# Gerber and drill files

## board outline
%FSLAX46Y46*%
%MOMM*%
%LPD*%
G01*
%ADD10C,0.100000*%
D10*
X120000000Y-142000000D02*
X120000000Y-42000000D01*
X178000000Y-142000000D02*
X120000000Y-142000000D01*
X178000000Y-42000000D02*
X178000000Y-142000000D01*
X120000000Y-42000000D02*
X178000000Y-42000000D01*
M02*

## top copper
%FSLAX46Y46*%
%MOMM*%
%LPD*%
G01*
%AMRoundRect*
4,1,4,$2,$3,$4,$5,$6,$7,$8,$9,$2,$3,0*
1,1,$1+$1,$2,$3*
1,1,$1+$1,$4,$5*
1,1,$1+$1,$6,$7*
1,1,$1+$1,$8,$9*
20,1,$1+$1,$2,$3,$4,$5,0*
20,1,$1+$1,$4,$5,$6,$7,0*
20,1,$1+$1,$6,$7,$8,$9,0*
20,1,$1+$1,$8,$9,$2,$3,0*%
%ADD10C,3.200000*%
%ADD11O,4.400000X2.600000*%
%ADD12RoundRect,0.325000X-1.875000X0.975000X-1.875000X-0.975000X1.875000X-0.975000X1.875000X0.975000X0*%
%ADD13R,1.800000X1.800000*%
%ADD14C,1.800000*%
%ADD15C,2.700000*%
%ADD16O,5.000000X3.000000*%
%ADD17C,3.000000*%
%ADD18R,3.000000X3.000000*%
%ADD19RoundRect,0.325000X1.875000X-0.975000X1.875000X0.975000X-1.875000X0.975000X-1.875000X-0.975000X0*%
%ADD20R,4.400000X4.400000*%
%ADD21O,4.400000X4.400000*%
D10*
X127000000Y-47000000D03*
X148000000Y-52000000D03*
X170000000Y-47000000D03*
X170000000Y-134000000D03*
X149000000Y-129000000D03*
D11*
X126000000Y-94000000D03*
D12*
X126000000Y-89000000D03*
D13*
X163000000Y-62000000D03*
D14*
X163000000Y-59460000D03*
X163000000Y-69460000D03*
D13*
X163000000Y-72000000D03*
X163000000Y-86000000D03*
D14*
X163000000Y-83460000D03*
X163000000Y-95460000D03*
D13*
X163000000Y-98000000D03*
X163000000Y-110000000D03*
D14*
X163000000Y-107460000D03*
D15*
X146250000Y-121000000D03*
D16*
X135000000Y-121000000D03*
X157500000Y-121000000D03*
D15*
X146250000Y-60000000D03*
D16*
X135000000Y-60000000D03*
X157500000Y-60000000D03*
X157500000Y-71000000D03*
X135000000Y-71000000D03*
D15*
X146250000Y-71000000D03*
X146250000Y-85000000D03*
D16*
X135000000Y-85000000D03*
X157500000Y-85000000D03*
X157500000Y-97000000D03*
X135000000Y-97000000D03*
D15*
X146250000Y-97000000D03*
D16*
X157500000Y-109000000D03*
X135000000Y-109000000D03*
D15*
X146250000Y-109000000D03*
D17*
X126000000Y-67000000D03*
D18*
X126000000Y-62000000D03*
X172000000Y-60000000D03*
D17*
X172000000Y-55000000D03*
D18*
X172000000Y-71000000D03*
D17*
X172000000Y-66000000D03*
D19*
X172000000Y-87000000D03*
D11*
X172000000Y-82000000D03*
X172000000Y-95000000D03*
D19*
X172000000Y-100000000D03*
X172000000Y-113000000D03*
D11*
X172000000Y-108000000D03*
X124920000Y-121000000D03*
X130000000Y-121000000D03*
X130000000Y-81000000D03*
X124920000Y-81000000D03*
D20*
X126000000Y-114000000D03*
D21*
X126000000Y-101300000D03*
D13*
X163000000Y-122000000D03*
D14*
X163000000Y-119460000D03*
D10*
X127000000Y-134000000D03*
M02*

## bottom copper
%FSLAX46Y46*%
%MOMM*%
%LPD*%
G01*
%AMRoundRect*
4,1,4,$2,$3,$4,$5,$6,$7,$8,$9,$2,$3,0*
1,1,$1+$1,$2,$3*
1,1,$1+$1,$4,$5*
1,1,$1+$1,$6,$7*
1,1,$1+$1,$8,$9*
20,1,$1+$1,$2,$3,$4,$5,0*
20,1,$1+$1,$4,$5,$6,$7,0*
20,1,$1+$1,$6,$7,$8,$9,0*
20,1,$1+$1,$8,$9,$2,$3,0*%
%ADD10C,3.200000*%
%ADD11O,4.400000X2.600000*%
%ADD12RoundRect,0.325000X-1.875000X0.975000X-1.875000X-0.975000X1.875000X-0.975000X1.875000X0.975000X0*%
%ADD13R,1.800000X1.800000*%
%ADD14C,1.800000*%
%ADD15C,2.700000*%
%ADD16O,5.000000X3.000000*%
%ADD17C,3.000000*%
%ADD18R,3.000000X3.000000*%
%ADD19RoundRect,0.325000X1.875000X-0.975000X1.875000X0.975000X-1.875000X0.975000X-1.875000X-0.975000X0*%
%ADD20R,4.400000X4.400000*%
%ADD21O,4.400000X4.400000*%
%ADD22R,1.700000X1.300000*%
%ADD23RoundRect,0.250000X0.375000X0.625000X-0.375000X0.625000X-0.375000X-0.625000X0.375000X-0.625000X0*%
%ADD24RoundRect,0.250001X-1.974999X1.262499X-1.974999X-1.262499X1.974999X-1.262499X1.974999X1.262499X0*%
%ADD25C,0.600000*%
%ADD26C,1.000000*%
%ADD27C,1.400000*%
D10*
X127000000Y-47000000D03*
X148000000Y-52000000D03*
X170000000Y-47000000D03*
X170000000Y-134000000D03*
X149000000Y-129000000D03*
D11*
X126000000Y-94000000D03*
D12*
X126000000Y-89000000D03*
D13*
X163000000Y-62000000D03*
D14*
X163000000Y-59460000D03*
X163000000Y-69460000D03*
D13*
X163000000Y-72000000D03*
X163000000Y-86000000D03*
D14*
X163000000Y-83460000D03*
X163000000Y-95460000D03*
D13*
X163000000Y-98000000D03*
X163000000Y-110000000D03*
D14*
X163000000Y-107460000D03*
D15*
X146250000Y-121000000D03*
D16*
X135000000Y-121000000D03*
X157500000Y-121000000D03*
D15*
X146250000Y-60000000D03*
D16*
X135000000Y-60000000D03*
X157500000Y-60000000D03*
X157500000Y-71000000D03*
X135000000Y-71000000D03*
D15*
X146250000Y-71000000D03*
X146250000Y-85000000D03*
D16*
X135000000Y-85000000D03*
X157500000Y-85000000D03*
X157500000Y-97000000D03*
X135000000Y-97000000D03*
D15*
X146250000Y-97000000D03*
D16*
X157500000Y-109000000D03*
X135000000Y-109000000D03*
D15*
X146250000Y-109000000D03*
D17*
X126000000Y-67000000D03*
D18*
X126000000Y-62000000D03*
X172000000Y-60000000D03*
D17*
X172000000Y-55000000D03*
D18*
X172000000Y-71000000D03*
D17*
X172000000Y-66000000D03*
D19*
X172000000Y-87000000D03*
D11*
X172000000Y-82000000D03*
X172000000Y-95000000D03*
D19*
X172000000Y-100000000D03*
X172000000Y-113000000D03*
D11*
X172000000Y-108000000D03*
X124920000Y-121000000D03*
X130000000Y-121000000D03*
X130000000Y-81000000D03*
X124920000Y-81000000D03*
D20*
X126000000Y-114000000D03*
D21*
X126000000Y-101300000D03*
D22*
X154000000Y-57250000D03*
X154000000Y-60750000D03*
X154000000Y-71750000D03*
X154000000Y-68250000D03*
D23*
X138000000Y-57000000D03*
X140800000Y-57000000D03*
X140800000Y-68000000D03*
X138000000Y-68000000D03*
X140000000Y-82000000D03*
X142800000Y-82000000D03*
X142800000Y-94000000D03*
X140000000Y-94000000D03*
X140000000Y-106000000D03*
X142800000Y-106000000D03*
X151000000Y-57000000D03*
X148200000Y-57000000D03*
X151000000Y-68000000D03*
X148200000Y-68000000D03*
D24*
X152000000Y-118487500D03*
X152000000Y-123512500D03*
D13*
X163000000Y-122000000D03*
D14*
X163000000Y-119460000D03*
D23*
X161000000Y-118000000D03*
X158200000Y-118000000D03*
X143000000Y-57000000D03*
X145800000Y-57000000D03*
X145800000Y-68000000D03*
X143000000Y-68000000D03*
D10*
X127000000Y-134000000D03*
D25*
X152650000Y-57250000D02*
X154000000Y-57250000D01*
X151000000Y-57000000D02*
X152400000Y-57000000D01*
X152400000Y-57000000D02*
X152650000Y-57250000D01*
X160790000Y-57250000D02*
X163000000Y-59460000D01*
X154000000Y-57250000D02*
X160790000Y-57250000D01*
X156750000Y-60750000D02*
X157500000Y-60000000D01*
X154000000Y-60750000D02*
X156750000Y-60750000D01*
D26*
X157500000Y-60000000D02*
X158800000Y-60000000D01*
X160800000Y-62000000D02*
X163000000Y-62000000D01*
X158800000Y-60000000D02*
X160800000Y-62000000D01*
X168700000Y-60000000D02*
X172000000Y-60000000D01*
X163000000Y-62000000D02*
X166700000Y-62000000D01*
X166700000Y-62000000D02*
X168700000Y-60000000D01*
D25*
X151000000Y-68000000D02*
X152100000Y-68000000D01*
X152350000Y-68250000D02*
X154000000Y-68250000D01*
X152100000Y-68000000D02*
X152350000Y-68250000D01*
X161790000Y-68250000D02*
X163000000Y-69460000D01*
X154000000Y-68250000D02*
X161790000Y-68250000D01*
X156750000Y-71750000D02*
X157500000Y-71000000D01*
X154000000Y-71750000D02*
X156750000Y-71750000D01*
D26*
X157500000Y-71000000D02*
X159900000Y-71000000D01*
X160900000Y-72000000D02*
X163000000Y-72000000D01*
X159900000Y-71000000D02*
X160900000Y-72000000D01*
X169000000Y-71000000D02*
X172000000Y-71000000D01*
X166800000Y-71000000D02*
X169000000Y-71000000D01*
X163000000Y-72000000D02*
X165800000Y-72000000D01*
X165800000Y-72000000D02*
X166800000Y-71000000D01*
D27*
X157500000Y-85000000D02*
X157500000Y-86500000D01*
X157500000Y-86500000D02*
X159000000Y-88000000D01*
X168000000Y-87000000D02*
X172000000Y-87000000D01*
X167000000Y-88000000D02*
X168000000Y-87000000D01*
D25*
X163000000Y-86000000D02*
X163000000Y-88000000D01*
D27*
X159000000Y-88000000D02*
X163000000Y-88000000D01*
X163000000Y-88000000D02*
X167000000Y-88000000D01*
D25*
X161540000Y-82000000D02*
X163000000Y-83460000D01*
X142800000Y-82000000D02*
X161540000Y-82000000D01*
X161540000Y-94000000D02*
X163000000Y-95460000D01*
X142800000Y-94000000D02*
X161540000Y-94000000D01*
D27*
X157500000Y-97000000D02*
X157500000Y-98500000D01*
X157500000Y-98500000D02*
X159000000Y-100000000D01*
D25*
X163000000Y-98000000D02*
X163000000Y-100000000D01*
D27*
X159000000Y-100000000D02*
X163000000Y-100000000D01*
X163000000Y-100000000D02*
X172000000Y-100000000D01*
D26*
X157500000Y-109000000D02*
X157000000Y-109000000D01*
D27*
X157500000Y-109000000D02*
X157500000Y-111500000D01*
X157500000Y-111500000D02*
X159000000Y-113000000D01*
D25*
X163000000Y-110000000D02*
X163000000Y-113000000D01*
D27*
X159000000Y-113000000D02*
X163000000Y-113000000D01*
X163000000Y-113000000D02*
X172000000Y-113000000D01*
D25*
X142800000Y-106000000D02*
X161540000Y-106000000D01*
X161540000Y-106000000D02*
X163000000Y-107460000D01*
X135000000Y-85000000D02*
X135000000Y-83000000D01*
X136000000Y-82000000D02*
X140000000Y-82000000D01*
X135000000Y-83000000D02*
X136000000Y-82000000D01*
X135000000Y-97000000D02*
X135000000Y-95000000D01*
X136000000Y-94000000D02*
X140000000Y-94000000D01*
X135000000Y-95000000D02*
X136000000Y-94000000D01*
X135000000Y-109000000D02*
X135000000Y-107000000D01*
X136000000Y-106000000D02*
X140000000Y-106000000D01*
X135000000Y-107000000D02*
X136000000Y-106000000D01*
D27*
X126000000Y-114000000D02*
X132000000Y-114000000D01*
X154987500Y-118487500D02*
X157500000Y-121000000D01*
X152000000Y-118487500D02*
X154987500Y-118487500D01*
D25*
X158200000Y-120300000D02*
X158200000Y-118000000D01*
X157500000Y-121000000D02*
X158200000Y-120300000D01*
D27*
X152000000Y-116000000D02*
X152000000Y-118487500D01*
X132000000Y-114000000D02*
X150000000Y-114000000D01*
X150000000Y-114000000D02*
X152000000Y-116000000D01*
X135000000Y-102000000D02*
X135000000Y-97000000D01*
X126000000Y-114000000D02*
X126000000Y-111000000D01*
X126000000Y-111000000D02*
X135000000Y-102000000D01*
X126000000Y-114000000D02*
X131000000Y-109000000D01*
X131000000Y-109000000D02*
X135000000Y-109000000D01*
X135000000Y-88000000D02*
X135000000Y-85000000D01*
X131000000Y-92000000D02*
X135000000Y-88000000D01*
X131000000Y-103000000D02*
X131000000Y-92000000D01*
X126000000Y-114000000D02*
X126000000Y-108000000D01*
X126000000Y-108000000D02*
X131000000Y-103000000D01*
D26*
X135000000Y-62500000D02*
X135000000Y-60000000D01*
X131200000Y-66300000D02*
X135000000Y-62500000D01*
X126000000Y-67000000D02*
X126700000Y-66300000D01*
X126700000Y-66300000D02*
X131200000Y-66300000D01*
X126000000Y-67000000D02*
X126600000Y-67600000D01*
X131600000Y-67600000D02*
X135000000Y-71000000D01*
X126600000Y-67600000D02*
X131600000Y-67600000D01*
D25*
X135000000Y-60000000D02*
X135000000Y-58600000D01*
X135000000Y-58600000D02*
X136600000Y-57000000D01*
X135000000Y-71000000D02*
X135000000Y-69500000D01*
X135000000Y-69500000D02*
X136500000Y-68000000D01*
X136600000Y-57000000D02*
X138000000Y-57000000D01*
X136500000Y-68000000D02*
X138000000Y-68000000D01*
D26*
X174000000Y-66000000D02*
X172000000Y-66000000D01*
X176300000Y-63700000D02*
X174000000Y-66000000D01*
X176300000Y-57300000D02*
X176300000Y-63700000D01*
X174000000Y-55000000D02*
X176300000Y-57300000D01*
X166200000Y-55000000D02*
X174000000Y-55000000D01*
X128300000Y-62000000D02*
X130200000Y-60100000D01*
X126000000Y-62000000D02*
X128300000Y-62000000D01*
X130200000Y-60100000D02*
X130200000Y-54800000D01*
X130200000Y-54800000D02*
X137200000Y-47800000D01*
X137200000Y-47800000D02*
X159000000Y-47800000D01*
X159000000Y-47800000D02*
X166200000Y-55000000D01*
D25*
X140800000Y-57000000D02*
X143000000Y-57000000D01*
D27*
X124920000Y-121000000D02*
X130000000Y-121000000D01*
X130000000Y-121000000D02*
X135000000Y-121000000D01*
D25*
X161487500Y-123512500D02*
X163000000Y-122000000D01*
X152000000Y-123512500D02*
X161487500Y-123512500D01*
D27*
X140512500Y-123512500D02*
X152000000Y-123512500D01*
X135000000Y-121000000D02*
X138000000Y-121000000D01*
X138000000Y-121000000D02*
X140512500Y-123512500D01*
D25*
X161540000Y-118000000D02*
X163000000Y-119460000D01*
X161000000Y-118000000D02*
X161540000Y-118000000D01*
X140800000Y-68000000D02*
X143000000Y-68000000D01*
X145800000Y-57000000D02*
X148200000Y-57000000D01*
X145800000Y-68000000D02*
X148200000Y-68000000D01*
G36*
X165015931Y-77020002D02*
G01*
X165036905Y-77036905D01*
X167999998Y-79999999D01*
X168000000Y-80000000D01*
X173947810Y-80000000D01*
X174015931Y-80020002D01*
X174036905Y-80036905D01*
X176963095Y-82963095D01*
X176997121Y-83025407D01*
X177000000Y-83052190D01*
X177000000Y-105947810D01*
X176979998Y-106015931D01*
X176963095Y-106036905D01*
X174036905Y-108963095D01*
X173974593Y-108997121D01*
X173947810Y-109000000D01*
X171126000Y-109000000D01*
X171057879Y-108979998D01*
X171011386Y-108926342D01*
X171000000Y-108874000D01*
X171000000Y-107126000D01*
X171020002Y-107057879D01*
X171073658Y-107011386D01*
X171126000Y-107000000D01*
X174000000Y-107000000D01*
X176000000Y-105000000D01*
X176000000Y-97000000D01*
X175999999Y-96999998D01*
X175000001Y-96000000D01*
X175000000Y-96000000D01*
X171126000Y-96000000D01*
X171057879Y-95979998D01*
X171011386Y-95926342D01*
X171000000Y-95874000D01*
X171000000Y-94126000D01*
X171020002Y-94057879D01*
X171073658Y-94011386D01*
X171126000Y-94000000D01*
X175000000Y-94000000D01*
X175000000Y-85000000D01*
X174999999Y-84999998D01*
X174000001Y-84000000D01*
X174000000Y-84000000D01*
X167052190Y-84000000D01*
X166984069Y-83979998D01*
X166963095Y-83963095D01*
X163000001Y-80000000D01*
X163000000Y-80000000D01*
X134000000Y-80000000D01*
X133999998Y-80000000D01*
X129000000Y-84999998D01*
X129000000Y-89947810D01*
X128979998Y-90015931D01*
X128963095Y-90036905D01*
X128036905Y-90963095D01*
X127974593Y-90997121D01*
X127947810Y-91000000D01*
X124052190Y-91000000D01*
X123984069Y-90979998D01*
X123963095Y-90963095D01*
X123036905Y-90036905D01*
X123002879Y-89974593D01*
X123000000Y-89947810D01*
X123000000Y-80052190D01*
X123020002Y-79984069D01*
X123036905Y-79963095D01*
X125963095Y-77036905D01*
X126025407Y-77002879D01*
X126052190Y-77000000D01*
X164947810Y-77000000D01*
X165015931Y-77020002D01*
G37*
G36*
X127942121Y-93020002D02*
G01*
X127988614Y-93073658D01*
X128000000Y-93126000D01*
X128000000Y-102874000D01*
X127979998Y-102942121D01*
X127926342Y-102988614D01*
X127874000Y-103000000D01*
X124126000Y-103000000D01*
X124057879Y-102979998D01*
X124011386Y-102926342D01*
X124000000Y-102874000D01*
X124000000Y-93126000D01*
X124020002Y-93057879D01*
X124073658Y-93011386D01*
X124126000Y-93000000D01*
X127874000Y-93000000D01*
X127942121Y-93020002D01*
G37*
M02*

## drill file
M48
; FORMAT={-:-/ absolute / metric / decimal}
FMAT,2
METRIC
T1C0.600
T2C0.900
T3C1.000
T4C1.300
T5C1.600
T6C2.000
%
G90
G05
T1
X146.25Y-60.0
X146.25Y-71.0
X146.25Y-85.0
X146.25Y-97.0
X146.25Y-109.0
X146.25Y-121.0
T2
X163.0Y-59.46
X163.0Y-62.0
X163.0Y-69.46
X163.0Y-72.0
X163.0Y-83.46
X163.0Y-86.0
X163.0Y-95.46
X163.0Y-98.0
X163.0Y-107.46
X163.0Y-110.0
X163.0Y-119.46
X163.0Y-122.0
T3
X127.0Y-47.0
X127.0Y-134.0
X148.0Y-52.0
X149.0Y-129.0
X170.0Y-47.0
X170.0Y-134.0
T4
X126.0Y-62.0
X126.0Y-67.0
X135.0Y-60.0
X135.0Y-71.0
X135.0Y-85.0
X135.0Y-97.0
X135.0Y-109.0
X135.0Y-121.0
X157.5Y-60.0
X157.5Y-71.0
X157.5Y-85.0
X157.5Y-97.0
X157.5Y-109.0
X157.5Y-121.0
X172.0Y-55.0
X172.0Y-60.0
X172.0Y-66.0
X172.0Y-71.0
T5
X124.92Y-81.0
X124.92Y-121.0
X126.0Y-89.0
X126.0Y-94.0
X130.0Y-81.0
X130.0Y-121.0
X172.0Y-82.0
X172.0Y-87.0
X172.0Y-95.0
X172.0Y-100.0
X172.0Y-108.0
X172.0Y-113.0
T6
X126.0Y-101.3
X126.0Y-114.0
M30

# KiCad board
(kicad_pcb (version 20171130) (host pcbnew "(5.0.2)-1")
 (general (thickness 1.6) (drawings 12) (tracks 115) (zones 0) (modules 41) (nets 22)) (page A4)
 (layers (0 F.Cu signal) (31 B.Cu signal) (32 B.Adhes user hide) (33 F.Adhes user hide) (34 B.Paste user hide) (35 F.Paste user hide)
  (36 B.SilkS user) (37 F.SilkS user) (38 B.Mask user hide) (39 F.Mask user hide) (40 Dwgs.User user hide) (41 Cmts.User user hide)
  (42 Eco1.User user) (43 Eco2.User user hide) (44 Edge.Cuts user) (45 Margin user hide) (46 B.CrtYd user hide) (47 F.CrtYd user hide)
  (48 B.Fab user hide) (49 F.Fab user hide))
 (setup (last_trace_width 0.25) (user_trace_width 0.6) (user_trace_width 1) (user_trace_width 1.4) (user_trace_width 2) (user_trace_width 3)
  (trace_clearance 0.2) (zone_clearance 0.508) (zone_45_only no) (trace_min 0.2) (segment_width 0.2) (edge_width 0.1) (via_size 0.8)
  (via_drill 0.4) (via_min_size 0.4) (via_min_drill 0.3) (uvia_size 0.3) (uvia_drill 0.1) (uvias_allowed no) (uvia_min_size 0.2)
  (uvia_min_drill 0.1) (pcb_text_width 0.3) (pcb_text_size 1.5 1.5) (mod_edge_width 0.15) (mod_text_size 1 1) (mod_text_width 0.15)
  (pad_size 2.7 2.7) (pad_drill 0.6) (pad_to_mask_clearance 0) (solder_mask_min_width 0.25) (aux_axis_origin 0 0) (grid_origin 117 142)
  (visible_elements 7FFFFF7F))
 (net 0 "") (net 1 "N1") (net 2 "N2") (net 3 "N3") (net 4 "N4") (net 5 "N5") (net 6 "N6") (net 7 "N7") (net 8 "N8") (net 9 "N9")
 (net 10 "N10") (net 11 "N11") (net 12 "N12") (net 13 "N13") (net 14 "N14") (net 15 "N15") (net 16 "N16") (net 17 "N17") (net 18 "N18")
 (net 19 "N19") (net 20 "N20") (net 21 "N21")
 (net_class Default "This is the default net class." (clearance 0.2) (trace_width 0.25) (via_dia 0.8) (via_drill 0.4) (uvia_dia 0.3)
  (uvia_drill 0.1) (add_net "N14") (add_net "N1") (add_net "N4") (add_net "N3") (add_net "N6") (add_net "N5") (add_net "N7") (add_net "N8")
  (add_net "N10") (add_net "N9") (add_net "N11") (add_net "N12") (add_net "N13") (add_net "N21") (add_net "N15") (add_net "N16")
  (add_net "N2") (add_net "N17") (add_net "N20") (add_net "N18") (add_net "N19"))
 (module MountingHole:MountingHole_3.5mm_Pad (layer F.Cu) (at 127 47)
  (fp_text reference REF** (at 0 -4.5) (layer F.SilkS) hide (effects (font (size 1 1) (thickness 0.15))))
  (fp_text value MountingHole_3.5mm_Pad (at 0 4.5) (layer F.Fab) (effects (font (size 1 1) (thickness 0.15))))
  (pad 1 thru_hole circle (at 0 0) (size 3.2 3.2) (drill 1) (layers *.Cu *.Mask)))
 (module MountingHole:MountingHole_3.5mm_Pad (layer F.Cu) (at 148 52)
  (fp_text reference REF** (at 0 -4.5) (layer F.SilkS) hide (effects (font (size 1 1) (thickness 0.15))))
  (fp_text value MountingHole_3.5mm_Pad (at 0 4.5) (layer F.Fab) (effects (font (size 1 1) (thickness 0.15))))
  (pad 1 thru_hole circle (at 0 0) (size 3.2 3.2) (drill 1) (layers *.Cu *.Mask)))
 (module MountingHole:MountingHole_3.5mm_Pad (layer F.Cu) (at 170 47)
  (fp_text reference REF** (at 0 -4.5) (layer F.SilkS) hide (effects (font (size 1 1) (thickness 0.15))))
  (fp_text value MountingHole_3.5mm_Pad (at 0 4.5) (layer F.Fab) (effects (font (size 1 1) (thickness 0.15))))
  (pad 1 thru_hole circle (at 0 0) (size 3.2 3.2) (drill 1) (layers *.Cu *.Mask)))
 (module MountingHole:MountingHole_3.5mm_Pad (layer F.Cu) (at 170 134)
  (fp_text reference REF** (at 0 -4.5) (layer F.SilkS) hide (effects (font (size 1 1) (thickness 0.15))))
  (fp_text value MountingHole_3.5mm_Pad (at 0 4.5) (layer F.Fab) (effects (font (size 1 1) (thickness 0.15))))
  (pad 1 thru_hole circle (at 0 0) (size 3.2 3.2) (drill 1) (layers *.Cu *.Mask)))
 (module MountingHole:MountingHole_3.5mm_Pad (layer F.Cu) (at 149 129)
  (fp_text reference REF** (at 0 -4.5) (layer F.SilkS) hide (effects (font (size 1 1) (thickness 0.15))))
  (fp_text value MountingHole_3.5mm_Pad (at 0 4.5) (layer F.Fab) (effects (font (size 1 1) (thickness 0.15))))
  (pad 1 thru_hole circle (at 0 0) (size 3.2 3.2) (drill 1) (layers *.Cu *.Mask)))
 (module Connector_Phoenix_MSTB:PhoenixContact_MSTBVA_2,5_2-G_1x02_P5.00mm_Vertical (layer F.Cu) (at 126 89 270)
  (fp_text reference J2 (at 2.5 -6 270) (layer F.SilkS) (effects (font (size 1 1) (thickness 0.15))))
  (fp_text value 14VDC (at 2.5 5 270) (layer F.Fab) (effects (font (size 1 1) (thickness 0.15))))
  (pad 2 thru_hole oval (at 5 0 270) (size 2.6 4.4) (drill 1.6) (layers *.Cu *.Mask) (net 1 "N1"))
  (pad 1 thru_hole roundrect (at 0 0 270) (size 2.6 4.4) (drill 1.6) (layers *.Cu *.Mask) (roundrect_rratio 0.125) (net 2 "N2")))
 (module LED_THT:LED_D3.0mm (layer F.Cu) (at 163 62 90)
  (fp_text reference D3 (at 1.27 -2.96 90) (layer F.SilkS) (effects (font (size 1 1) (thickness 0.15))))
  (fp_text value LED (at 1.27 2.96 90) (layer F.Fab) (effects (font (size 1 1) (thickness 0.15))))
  (pad 1 thru_hole rect (at 0 0 90) (size 1.8 1.8) (drill 0.9) (layers *.Cu *.Mask) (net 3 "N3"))
  (pad 2 thru_hole circle (at 2.54 0 90) (size 1.8 1.8) (drill 0.9) (layers *.Cu *.Mask) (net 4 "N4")))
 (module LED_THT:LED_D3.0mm (layer F.Cu) (at 163 72 90)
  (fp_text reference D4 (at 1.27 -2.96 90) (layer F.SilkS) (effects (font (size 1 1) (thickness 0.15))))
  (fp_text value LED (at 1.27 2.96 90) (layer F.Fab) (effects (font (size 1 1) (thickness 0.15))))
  (pad 2 thru_hole circle (at 2.54 0 90) (size 1.8 1.8) (drill 0.9) (layers *.Cu *.Mask) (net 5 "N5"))
  (pad 1 thru_hole rect (at 0 0 90) (size 1.8 1.8) (drill 0.9) (layers *.Cu *.Mask) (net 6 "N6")))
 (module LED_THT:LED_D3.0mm (layer F.Cu) (at 163 86 90)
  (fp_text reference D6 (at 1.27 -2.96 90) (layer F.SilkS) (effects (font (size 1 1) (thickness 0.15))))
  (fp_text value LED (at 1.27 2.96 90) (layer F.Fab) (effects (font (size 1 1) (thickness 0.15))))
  (pad 1 thru_hole rect (at 0 0 90) (size 1.8 1.8) (drill 0.9) (layers *.Cu *.Mask) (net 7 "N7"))
  (pad 2 thru_hole circle (at 2.54 0 90) (size 1.8 1.8) (drill 0.9) (layers *.Cu *.Mask) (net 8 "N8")))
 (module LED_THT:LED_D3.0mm (layer F.Cu) (at 163 98 90)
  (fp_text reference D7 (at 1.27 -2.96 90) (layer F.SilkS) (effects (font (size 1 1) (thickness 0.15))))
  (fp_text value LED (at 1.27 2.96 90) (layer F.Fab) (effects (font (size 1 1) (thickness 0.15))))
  (pad 2 thru_hole circle (at 2.54 0 90) (size 1.8 1.8) (drill 0.9) (layers *.Cu *.Mask) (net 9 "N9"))
  (pad 1 thru_hole rect (at 0 0 90) (size 1.8 1.8) (drill 0.9) (layers *.Cu *.Mask) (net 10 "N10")))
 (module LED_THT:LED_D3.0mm (layer F.Cu) (at 163 110 90)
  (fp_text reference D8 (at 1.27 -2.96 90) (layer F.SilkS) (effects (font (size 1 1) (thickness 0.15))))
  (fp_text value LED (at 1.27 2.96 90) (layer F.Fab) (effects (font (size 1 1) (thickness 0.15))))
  (pad 1 thru_hole rect (at 0 0 90) (size 1.8 1.8) (drill 0.9) (layers *.Cu *.Mask) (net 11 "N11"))
  (pad 2 thru_hole circle (at 2.54 0 90) (size 1.8 1.8) (drill 0.9) (layers *.Cu *.Mask) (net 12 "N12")))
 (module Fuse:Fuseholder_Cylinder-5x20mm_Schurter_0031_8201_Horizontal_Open (layer F.Cu) (at 157.5 121 180)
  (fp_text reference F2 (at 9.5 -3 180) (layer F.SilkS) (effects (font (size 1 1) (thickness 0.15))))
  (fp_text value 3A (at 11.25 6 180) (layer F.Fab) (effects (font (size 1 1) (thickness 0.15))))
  (pad "" thru_hole circle (at 11.25 0 180) (size 2.7 2.7) (drill 0.6) (layers *.Cu *.Mask))
  (pad 2 thru_hole oval (at 22.5 0 180) (size 5 3) (drill 1.3) (layers *.Cu *.Mask) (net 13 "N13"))
  (pad 1 thru_hole oval (at 0 0 180) (size 5 3) (drill 1.3) (layers *.Cu *.Mask) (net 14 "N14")))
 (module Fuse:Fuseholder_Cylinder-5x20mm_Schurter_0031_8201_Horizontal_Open (layer F.Cu) (at 157.5 60 180)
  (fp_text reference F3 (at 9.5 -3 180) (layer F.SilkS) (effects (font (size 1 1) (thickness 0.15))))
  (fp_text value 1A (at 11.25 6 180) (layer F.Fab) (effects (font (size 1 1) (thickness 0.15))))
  (pad "" thru_hole circle (at 11.25 0 180) (size 2.7 2.7) (drill 0.6) (layers *.Cu *.Mask))
  (pad 2 thru_hole oval (at 22.5 0 180) (size 5 3) (drill 1.3) (layers *.Cu *.Mask) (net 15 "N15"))
  (pad 1 thru_hole oval (at 0 0 180) (size 5 3) (drill 1.3) (layers *.Cu *.Mask) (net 3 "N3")))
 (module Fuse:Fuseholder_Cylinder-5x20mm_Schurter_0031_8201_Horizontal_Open (layer F.Cu) (at 157.5 71 180)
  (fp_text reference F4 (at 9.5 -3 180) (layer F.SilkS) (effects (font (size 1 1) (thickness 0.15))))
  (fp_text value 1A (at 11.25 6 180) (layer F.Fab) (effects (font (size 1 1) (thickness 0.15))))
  (pad 1 thru_hole oval (at 0 0 180) (size 5 3) (drill 1.3) (layers *.Cu *.Mask) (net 6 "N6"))
  (pad 2 thru_hole oval (at 22.5 0 180) (size 5 3) (drill 1.3) (layers *.Cu *.Mask) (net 15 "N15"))
  (pad "" thru_hole circle (at 11.25 0 180) (size 2.7 2.7) (drill 0.6) (layers *.Cu *.Mask)))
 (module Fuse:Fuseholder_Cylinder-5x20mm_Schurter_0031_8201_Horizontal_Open (layer F.Cu) (at 157.5 85 180)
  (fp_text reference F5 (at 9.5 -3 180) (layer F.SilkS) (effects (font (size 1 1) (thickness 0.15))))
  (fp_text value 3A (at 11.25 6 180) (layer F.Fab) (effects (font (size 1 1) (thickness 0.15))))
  (pad "" thru_hole circle (at 11.25 0 180) (size 2.7 2.7) (drill 0.6) (layers *.Cu *.Mask))
  (pad 2 thru_hole oval (at 22.5 0 180) (size 5 3) (drill 1.3) (layers *.Cu *.Mask) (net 14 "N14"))
  (pad 1 thru_hole oval (at 0 0 180) (size 5 3) (drill 1.3) (layers *.Cu *.Mask) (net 7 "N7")))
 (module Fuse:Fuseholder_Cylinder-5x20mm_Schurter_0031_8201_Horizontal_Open (layer F.Cu) (at 157.5 97 180)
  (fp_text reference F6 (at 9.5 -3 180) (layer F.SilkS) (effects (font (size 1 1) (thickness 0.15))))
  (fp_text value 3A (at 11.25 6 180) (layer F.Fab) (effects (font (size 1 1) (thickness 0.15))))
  (pad 1 thru_hole oval (at 0 0 180) (size 5 3) (drill 1.3) (layers *.Cu *.Mask) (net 10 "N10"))
  (pad 2 thru_hole oval (at 22.5 0 180) (size 5 3) (drill 1.3) (layers *.Cu *.Mask) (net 14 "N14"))
  (pad "" thru_hole circle (at 11.25 0 180) (size 2.7 2.7) (drill 0.6) (layers *.Cu *.Mask)))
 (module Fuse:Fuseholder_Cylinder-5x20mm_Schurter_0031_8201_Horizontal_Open (layer F.Cu) (at 157.5 109 180)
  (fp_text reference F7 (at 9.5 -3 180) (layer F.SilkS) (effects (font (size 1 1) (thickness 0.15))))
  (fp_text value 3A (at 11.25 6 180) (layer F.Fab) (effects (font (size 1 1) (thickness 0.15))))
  (pad 1 thru_hole oval (at 0 0 180) (size 5 3) (drill 1.3) (layers *.Cu *.Mask) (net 11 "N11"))
  (pad 2 thru_hole oval (at 22.5 0 180) (size 5 3) (drill 1.3) (layers *.Cu *.Mask) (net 14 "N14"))
  (pad "" thru_hole circle (at 11.25 0 180) (size 2.7 2.7) (drill 0.6) (layers *.Cu *.Mask)))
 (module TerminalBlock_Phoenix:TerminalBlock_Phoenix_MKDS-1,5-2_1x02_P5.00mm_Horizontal (layer F.Cu) (at 126 62 270)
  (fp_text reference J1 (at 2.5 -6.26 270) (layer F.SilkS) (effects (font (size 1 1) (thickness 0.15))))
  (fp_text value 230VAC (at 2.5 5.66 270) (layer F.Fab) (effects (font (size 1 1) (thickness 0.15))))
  (pad 2 thru_hole circle (at 5 0 270) (size 3 3) (drill 1.3) (layers *.Cu *.Mask) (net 15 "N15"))
  (pad 1 thru_hole rect (at 0 0 270) (size 3 3) (drill 1.3) (layers *.Cu *.Mask) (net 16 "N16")))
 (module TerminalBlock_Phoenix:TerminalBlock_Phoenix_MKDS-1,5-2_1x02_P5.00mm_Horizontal (layer F.Cu) (at 172 60 90)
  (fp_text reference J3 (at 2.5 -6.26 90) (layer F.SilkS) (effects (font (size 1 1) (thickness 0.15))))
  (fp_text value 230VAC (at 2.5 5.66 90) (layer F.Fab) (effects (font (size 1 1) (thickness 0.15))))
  (pad 1 thru_hole rect (at 0 0 90) (size 3 3) (drill 1.3) (layers *.Cu *.Mask) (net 3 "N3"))
  (pad 2 thru_hole circle (at 5 0 90) (size 3 3) (drill 1.3) (layers *.Cu *.Mask) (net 16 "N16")))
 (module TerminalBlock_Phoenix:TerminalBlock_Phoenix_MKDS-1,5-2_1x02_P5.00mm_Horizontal (layer F.Cu) (at 172 71 90)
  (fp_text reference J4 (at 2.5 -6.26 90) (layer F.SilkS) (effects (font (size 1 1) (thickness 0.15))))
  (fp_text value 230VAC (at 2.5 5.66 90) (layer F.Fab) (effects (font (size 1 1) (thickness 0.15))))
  (pad 1 thru_hole rect (at 0 0 90) (size 3 3) (drill 1.3) (layers *.Cu *.Mask) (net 6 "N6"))
  (pad 2 thru_hole circle (at 5 0 90) (size 3 3) (drill 1.3) (layers *.Cu *.Mask) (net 16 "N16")))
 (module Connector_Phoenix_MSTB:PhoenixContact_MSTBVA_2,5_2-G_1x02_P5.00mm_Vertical (layer F.Cu) (at 172 87 90)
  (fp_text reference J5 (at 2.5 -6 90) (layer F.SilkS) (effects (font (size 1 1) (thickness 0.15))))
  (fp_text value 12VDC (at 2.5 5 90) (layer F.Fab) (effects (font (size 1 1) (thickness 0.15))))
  (pad 1 thru_hole roundrect (at 0 0 90) (size 2.6 4.4) (drill 1.6) (layers *.Cu *.Mask) (roundrect_rratio 0.125) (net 7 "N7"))
  (pad 2 thru_hole oval (at 5 0 90) (size 2.6 4.4) (drill 1.6) (layers *.Cu *.Mask) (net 2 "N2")))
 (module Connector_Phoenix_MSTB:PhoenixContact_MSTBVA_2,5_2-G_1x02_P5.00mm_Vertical (layer F.Cu) (at 172 100 90)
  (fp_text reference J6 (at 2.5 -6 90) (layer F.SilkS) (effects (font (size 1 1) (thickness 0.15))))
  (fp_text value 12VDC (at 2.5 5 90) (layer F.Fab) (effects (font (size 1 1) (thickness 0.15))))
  (pad 2 thru_hole oval (at 5 0 90) (size 2.6 4.4) (drill 1.6) (layers *.Cu *.Mask) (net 2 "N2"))
  (pad 1 thru_hole roundrect (at 0 0 90) (size 2.6 4.4) (drill 1.6) (layers *.Cu *.Mask) (roundrect_rratio 0.125) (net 10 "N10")))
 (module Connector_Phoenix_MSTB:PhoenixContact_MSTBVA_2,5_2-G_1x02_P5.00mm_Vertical (layer F.Cu) (at 172 113 90)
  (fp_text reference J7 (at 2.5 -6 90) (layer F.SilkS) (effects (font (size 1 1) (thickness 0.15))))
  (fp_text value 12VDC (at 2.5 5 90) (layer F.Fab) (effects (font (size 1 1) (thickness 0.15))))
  (pad 1 thru_hole roundrect (at 0 0 90) (size 2.6 4.4) (drill 1.6) (layers *.Cu *.Mask) (roundrect_rratio 0.125) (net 11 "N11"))
  (pad 2 thru_hole oval (at 5 0 90) (size 2.6 4.4) (drill 1.6) (layers *.Cu *.Mask) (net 2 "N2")))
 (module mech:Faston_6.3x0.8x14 (layer F.Cu) (at 127.46 121)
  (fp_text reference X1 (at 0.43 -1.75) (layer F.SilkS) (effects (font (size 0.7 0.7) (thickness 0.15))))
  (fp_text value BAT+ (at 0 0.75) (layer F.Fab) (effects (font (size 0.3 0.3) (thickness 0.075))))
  (pad 1 thru_hole oval (at -2.54 0) (size 4.4 2.6) (drill 1.6) (layers *.Cu *.Mask) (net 13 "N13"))
  (pad 1 thru_hole oval (at 2.54 0) (size 4.4 2.6) (drill 1.6) (layers *.Cu *.Mask) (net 13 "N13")))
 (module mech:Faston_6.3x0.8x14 (layer F.Cu) (at 127.46 81)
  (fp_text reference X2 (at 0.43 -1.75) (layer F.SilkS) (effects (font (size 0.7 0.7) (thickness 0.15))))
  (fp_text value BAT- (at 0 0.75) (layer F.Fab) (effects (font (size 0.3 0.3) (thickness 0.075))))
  (pad 1 thru_hole oval (at 2.54 0) (size 4.4 2.6) (drill 1.6) (layers *.Cu *.Mask) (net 2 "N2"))
  (pad 1 thru_hole oval (at -2.54 0) (size 4.4 2.6) (drill 1.6) (layers *.Cu *.Mask) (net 2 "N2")))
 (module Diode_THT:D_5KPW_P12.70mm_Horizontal (layer F.Cu) (at 126 114 90)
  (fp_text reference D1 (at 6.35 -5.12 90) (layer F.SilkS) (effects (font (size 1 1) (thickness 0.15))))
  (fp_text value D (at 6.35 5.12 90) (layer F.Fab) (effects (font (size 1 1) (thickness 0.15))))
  (pad 1 thru_hole rect (at 0 0 90) (size 4.4 4.4) (drill 2) (layers *.Cu *.Mask) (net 14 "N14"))
  (pad 2 thru_hole oval (at 12.7 0 90) (size 4.4 4.4) (drill 2) (layers *.Cu *.Mask) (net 1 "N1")))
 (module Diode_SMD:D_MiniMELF (layer B.Cu) (at 154 59 270)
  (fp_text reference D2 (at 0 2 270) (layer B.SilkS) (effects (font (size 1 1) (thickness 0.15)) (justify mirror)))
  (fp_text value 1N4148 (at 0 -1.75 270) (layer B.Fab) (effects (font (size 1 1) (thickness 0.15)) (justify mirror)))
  (pad 1 smd rect (at -1.75 0 270) (size 1.3 1.7) (layers B.Cu B.Paste B.Mask) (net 4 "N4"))
  (pad 2 smd rect (at 1.75 0 270) (size 1.3 1.7) (layers B.Cu B.Paste B.Mask) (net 3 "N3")))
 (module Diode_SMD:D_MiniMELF (layer B.Cu) (at 154 70 270)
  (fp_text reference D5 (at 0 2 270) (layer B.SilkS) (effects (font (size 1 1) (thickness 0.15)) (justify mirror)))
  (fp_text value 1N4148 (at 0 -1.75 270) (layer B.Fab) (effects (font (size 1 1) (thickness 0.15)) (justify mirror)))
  (pad 2 smd rect (at 1.75 0 270) (size 1.3 1.7) (layers B.Cu B.Paste B.Mask) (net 6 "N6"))
  (pad 1 smd rect (at -1.75 0 270) (size 1.3 1.7) (layers B.Cu B.Paste B.Mask) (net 5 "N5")))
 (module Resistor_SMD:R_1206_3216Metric (layer B.Cu) (at 139.4 57 180)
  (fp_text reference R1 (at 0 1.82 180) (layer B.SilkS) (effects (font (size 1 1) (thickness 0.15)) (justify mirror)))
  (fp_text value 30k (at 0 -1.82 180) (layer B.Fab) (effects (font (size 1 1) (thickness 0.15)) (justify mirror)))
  (pad 2 smd roundrect (at 1.4 0 180) (size 1.25 1.75) (layers B.Cu B.Paste B.Mask) (roundrect_rratio 0.2) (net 15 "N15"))
  (pad 1 smd roundrect (at -1.4 0 180) (size 1.25 1.75) (layers B.Cu B.Paste B.Mask) (roundrect_rratio 0.2) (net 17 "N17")))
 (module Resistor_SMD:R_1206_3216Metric (layer B.Cu) (at 139.4 68 180)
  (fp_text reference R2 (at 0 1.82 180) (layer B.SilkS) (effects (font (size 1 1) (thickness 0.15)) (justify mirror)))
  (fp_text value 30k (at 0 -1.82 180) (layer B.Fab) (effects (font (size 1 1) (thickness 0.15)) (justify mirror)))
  (pad 1 smd roundrect (at -1.4 0 180) (size 1.25 1.75) (layers B.Cu B.Paste B.Mask) (roundrect_rratio 0.2) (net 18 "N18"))
  (pad 2 smd roundrect (at 1.4 0 180) (size 1.25 1.75) (layers B.Cu B.Paste B.Mask) (roundrect_rratio 0.2) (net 15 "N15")))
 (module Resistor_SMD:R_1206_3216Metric (layer B.Cu) (at 141.4 82 180)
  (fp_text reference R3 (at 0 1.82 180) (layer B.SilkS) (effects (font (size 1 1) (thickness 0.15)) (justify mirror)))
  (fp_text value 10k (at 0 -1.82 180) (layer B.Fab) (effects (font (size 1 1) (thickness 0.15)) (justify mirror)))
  (pad 2 smd roundrect (at 1.4 0 180) (size 1.25 1.75) (layers B.Cu B.Paste B.Mask) (roundrect_rratio 0.2) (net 14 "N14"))
  (pad 1 smd roundrect (at -1.4 0 180) (size 1.25 1.75) (layers B.Cu B.Paste B.Mask) (roundrect_rratio 0.2) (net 8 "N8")))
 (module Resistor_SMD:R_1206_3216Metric (layer B.Cu) (at 141.4 94 180)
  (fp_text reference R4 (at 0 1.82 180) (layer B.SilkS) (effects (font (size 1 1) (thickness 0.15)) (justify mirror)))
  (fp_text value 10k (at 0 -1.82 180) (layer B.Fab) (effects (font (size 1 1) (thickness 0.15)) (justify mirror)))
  (pad 1 smd roundrect (at -1.4 0 180) (size 1.25 1.75) (layers B.Cu B.Paste B.Mask) (roundrect_rratio 0.2) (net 9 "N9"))
  (pad 2 smd roundrect (at 1.4 0 180) (size 1.25 1.75) (layers B.Cu B.Paste B.Mask) (roundrect_rratio 0.2) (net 14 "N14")))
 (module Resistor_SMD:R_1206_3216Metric (layer B.Cu) (at 141.4 106 180)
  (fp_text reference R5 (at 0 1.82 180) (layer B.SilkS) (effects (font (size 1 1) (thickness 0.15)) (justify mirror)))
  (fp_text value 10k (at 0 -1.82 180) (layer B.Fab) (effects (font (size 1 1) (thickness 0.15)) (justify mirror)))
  (pad 2 smd roundrect (at 1.4 0 180) (size 1.25 1.75) (layers B.Cu B.Paste B.Mask) (roundrect_rratio 0.2) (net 14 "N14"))
  (pad 1 smd roundrect (at -1.4 0 180) (size 1.25 1.75) (layers B.Cu B.Paste B.Mask) (roundrect_rratio 0.2) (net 12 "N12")))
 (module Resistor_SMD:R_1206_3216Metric (layer B.Cu) (at 149.6 57 180)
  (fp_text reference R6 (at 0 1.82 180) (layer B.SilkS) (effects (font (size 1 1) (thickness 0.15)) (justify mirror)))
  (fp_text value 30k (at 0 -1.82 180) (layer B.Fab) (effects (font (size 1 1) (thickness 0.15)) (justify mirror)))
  (pad 1 smd roundrect (at -1.4 0 180) (size 1.25 1.75) (layers B.Cu B.Paste B.Mask) (roundrect_rratio 0.2) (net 4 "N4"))
  (pad 2 smd roundrect (at 1.4 0 180) (size 1.25 1.75) (layers B.Cu B.Paste B.Mask) (roundrect_rratio 0.2) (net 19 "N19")))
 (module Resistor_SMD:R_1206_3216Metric (layer B.Cu) (at 149.6 68 180)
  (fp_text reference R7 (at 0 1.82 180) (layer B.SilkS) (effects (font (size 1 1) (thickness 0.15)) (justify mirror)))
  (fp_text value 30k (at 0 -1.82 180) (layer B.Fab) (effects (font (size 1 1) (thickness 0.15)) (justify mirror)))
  (pad 1 smd roundrect (at -1.4 0 180) (size 1.25 1.75) (layers B.Cu B.Paste B.Mask) (roundrect_rratio 0.2) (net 5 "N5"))
  (pad 2 smd roundrect (at 1.4 0 180) (size 1.25 1.75) (layers B.Cu B.Paste B.Mask) (roundrect_rratio 0.2) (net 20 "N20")))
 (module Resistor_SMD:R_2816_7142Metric (layer B.Cu) (at 152 121 270)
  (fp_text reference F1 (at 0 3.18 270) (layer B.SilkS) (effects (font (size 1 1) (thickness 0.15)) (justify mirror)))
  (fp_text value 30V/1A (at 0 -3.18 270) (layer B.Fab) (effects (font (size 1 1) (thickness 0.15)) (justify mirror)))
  (pad 1 smd roundrect (at -2.5125 0 270) (size 3.025 4.45) (layers B.Cu B.Paste B.Mask) (roundrect_rratio 0.082645) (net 14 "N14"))
  (pad 2 smd roundrect (at 2.5125 0 270) (size 3.025 4.45) (layers B.Cu B.Paste B.Mask) (roundrect_rratio 0.082645) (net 13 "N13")))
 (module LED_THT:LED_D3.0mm (layer F.Cu) (at 163 122 90)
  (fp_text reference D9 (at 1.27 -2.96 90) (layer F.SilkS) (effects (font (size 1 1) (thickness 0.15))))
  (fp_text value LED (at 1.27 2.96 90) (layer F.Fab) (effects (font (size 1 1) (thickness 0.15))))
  (pad 1 thru_hole rect (at 0 0 90) (size 1.8 1.8) (drill 0.9) (layers *.Cu *.Mask) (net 13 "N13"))
  (pad 2 thru_hole circle (at 2.54 0 90) (size 1.8 1.8) (drill 0.9) (layers *.Cu *.Mask) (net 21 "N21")))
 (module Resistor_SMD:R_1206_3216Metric (layer B.Cu) (at 159.6 118 180)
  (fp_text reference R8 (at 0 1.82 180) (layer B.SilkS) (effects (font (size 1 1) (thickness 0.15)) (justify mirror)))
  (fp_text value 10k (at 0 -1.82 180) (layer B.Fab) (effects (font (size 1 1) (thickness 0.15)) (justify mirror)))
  (pad 1 smd roundrect (at -1.4 0 180) (size 1.25 1.75) (layers B.Cu B.Paste B.Mask) (roundrect_rratio 0.2) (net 21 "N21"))
  (pad 2 smd roundrect (at 1.4 0 180) (size 1.25 1.75) (layers B.Cu B.Paste B.Mask) (roundrect_rratio 0.2) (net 14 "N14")))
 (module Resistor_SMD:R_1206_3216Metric (layer B.Cu) (at 144.4 57 180)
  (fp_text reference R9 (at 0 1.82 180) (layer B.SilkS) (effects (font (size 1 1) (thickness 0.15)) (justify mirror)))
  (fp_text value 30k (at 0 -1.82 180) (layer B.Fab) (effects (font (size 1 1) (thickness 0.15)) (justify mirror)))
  (pad 2 smd roundrect (at 1.4 0 180) (size 1.25 1.75) (layers B.Cu B.Paste B.Mask) (roundrect_rratio 0.2) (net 17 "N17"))
  (pad 1 smd roundrect (at -1.4 0 180) (size 1.25 1.75) (layers B.Cu B.Paste B.Mask) (roundrect_rratio 0.2) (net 19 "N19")))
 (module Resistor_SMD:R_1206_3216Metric (layer B.Cu) (at 144.4 68 180)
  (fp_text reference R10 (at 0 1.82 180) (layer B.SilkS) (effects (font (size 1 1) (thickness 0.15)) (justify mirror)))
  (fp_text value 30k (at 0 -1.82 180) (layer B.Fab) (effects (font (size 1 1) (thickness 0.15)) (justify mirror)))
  (pad 1 smd roundrect (at -1.4 0 180) (size 1.25 1.75) (layers B.Cu B.Paste B.Mask) (roundrect_rratio 0.2) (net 20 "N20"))
  (pad 2 smd roundrect (at 1.4 0 180) (size 1.25 1.75) (layers B.Cu B.Paste B.Mask) (roundrect_rratio 0.2) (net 18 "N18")))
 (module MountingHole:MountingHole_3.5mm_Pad (layer F.Cu) (at 127 134)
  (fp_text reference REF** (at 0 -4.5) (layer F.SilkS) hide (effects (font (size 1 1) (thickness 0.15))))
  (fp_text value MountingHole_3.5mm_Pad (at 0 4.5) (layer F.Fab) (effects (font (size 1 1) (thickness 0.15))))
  (pad 1 thru_hole circle (at 0 0) (size 3.2 3.2) (drill 1) (layers *.Cu *.Mask)))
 (gr_line (start 120 142) (end 120 42) (layer Edge.Cuts) (width 0.1))
 (gr_line (start 178 142) (end 120 142) (layer Edge.Cuts) (width 0.1))
 (gr_line (start 178 42) (end 178 142) (layer Edge.Cuts) (width 0.1))
 (gr_line (start 120 42) (end 178 42) (layer Edge.Cuts) (width 0.1))
 (segment (start 152.65 57.25) (end 154 57.25) (width 0.6) (layer B.Cu) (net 4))
 (segment (start 151 57) (end 152.4 57) (width 0.6) (layer B.Cu) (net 4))
 (segment (start 152.4 57) (end 152.65 57.25) (width 0.6) (layer B.Cu) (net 4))
 (segment (start 160.79 57.25) (end 163 59.46) (width 0.6) (layer B.Cu) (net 4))
 (segment (start 154 57.25) (end 160.79 57.25) (width 0.6) (layer B.Cu) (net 4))
 (segment (start 156.75 60.75) (end 157.5 60) (width 0.6) (layer B.Cu) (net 3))
 (segment (start 154 60.75) (end 156.75 60.75) (width 0.6) (layer B.Cu) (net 3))
 (segment (start 157.5 60) (end 158.8 60) (width 1) (layer B.Cu) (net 3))
 (segment (start 160.8 62) (end 163 62) (width 1) (layer B.Cu) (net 3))
 (segment (start 158.8 60) (end 160.8 62) (width 1) (layer B.Cu) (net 3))
 (segment (start 168.7 60) (end 172 60) (width 1) (layer B.Cu) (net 3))
 (segment (start 163 62) (end 166.7 62) (width 1) (layer B.Cu) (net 3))
 (segment (start 166.7 62) (end 168.7 60) (width 1) (layer B.Cu) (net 3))
 (segment (start 151 68) (end 152.1 68) (width 0.6) (layer B.Cu) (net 5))
 (segment (start 152.35 68.25) (end 154 68.25) (width 0.6) (layer B.Cu) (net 5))
 (segment (start 152.1 68) (end 152.35 68.25) (width 0.6) (layer B.Cu) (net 5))
 (segment (start 161.79 68.25) (end 163 69.46) (width 0.6) (layer B.Cu) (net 5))
 (segment (start 154 68.25) (end 161.79 68.25) (width 0.6) (layer B.Cu) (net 5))
 (segment (start 156.75 71.75) (end 157.5 71) (width 0.6) (layer B.Cu) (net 6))
 (segment (start 154 71.75) (end 156.75 71.75) (width 0.6) (layer B.Cu) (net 6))
 (segment (start 157.5 71) (end 159.9 71) (width 1) (layer B.Cu) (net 6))
 (segment (start 160.9 72) (end 163 72) (width 1) (layer B.Cu) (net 6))
 (segment (start 159.9 71) (end 160.9 72) (width 1) (layer B.Cu) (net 6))
 (segment (start 169 71) (end 172 71) (width 1) (layer B.Cu) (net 6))
 (segment (start 166.8 71) (end 169 71) (width 1) (layer B.Cu) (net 6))
 (segment (start 163 72) (end 165.8 72) (width 1) (layer B.Cu) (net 6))
 (segment (start 165.8 72) (end 166.8 71) (width 1) (layer B.Cu) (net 6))
 (segment (start 157.5 85) (end 157.5 86.5) (width 1.4) (layer B.Cu) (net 7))
 (segment (start 157.5 86.5) (end 159 88) (width 1.4) (layer B.Cu) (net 7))
 (segment (start 168 87) (end 172 87) (width 1.4) (layer B.Cu) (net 7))
 (segment (start 167 88) (end 168 87) (width 1.4) (layer B.Cu) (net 7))
 (segment (start 163 86) (end 163 88) (width 0.6) (layer B.Cu) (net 7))
 (segment (start 159 88) (end 163 88) (width 1.4) (layer B.Cu) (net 7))
 (segment (start 163 88) (end 167 88) (width 1.4) (layer B.Cu) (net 7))
 (segment (start 161.54 82) (end 163 83.46) (width 0.6) (layer B.Cu) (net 8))
 (segment (start 142.8 82) (end 161.54 82) (width 0.6) (layer B.Cu) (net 8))
 (segment (start 161.54 94) (end 163 95.46) (width 0.6) (layer B.Cu) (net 9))
 (segment (start 142.8 94) (end 161.54 94) (width 0.6) (layer B.Cu) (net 9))
 (segment (start 157.5 97) (end 157.5 98.5) (width 1.4) (layer B.Cu) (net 10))
 (segment (start 157.5 98.5) (end 159 100) (width 1.4) (layer B.Cu) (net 10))
 (segment (start 163 98) (end 163 100) (width 0.6) (layer B.Cu) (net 10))
 (segment (start 159 100) (end 163 100) (width 1.4) (layer B.Cu) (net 10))
 (segment (start 163 100) (end 172 100) (width 1.4) (layer B.Cu) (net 10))
 (segment (start 157.5 109) (end 157 109) (width 1) (layer B.Cu) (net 11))
 (segment (start 157.5 109) (end 157.5 111.5) (width 1.4) (layer B.Cu) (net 11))
 (segment (start 157.5 111.5) (end 159 113) (width 1.4) (layer B.Cu) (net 11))
 (segment (start 163 110) (end 163 113) (width 0.6) (layer B.Cu) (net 11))
 (segment (start 159 113) (end 163 113) (width 1.4) (layer B.Cu) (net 11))
 (segment (start 163 113) (end 172 113) (width 1.4) (layer B.Cu) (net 11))
 (segment (start 142.8 106) (end 161.54 106) (width 0.6) (layer B.Cu) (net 12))
 (segment (start 161.54 106) (end 163 107.46) (width 0.6) (layer B.Cu) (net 12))
 (segment (start 135 85) (end 135 83) (width 0.6) (layer B.Cu) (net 14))
 (segment (start 136 82) (end 140 82) (width 0.6) (layer B.Cu) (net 14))
 (segment (start 135 83) (end 136 82) (width 0.6) (layer B.Cu) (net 14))
 (segment (start 135 97) (end 135 95) (width 0.6) (layer B.Cu) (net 14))
 (segment (start 136 94) (end 140 94) (width 0.6) (layer B.Cu) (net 14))
 (segment (start 135 95) (end 136 94) (width 0.6) (layer B.Cu) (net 14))
 (segment (start 135 109) (end 135 107) (width 0.6) (layer B.Cu) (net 14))
 (segment (start 136 106) (end 140 106) (width 0.6) (layer B.Cu) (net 14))
 (segment (start 135 107) (end 136 106) (width 0.6) (layer B.Cu) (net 14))
 (segment (start 126 114) (end 132 114) (width 1.4) (layer B.Cu) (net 14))
 (segment (start 154.9875 118.4875) (end 157.5 121) (width 1.4) (layer B.Cu) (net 14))
 (segment (start 152 118.4875) (end 154.9875 118.4875) (width 1.4) (layer B.Cu) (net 14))
 (segment (start 158.2 120.3) (end 158.2 118) (width 0.6) (layer B.Cu) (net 14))
 (segment (start 157.5 121) (end 158.2 120.3) (width 0.6) (layer B.Cu) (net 14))
 (segment (start 152 116) (end 152 118.4875) (width 1.4) (layer B.Cu) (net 14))
 (segment (start 132 114) (end 150 114) (width 1.4) (layer B.Cu) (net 14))
 (segment (start 150 114) (end 152 116) (width 1.4) (layer B.Cu) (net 14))
 (segment (start 135 102) (end 135 97) (width 1.4) (layer B.Cu) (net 14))
 (segment (start 126 114) (end 126 111) (width 1.4) (layer B.Cu) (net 14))
 (segment (start 126 111) (end 135 102) (width 1.4) (layer B.Cu) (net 14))
 (segment (start 126 114) (end 131 109) (width 1.4) (layer B.Cu) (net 14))
 (segment (start 131 109) (end 135 109) (width 1.4) (layer B.Cu) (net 14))
 (segment (start 135 88) (end 135 85) (width 1.4) (layer B.Cu) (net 14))
 (segment (start 131 92) (end 135 88) (width 1.4) (layer B.Cu) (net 14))
 (segment (start 131 103) (end 131 92) (width 1.4) (layer B.Cu) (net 14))
 (segment (start 126 114) (end 126 108) (width 1.4) (layer B.Cu) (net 14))
 (segment (start 126 108) (end 131 103) (width 1.4) (layer B.Cu) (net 14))
 (segment (start 135 62.5) (end 135 60) (width 1) (layer B.Cu) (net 15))
 (segment (start 131.2 66.3) (end 135 62.5) (width 1) (layer B.Cu) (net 15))
 (segment (start 126 67) (end 126.7 66.3) (width 1) (layer B.Cu) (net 15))
 (segment (start 126.7 66.3) (end 131.2 66.3) (width 1) (layer B.Cu) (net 15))
 (segment (start 126 67) (end 126.6 67.6) (width 1) (layer B.Cu) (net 15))
 (segment (start 131.6 67.6) (end 135 71) (width 1) (layer B.Cu) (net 15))
 (segment (start 126.6 67.6) (end 131.6 67.6) (width 1) (layer B.Cu) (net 15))
 (segment (start 135 60) (end 135 58.6) (width 0.6) (layer B.Cu) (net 15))
 (segment (start 135 58.6) (end 136.6 57) (width 0.6) (layer B.Cu) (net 15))
 (segment (start 135 71) (end 135 69.5) (width 0.6) (layer B.Cu) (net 15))
 (segment (start 135 69.5) (end 136.5 68) (width 0.6) (layer B.Cu) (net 15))
 (segment (start 136.6 57) (end 138 57) (width 0.6) (layer B.Cu) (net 15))
 (segment (start 136.5 68) (end 138 68) (width 0.6) (layer B.Cu) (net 15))
 (segment (start 174 66) (end 172 66) (width 1) (layer B.Cu) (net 16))
 (segment (start 176.3 63.7) (end 174 66) (width 1) (layer B.Cu) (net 16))
 (segment (start 176.3 57.3) (end 176.3 63.7) (width 1) (layer B.Cu) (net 16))
 (segment (start 174 55) (end 176.3 57.3) (width 1) (layer B.Cu) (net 16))
 (segment (start 166.2 55) (end 174 55) (width 1) (layer B.Cu) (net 16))
 (segment (start 128.3 62) (end 130.2 60.1) (width 1) (layer B.Cu) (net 16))
 (segment (start 126 62) (end 128.3 62) (width 1) (layer B.Cu) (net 16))
 (segment (start 130.2 60.1) (end 130.2 54.8) (width 1) (layer B.Cu) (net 16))
 (segment (start 130.2 54.8) (end 137.2 47.8) (width 1) (layer B.Cu) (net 16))
 (segment (start 137.2 47.8) (end 159 47.8) (width 1) (layer B.Cu) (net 16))
 (segment (start 159 47.8) (end 166.2 55) (width 1) (layer B.Cu) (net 16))
 (segment (start 140.8 57) (end 143 57) (width 0.6) (layer B.Cu) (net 17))
 (segment (start 124.92 121) (end 130 121) (width 1.4) (layer B.Cu) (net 13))
 (segment (start 130 121) (end 135 121) (width 1.4) (layer B.Cu) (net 13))
 (segment (start 161.4875 123.5125) (end 163 122) (width 0.6) (layer B.Cu) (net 13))
 (segment (start 152 123.5125) (end 161.4875 123.5125) (width 0.6) (layer B.Cu) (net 13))
 (segment (start 140.5125 123.5125) (end 152 123.5125) (width 1.4) (layer B.Cu) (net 13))
 (segment (start 135 121) (end 138 121) (width 1.4) (layer B.Cu) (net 13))
 (segment (start 138 121) (end 140.5125 123.5125) (width 1.4) (layer B.Cu) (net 13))
 (segment (start 161.54 118) (end 163 119.46) (width 0.6) (layer B.Cu) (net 21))
 (segment (start 161 118) (end 161.54 118) (width 0.6) (layer B.Cu) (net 21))
 (segment (start 140.8 68) (end 143 68) (width 0.6) (layer B.Cu) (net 18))
 (segment (start 145.8 57) (end 148.2 57) (width 0.6) (layer B.Cu) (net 19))
 (segment (start 145.8 68) (end 148.2 68) (width 0.6) (layer B.Cu) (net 20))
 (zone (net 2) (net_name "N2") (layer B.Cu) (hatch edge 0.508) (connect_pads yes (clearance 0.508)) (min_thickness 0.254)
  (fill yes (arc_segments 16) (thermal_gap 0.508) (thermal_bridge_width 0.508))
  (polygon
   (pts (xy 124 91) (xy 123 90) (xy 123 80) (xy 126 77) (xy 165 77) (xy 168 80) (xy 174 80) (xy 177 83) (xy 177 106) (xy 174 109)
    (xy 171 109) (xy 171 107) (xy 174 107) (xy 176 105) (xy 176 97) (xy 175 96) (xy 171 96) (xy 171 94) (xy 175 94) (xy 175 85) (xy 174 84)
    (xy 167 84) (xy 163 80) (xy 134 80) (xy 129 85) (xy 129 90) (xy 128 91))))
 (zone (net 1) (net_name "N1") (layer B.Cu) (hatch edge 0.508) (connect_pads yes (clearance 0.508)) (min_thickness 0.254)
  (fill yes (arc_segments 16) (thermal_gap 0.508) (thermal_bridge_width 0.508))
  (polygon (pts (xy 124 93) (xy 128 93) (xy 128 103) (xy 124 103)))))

